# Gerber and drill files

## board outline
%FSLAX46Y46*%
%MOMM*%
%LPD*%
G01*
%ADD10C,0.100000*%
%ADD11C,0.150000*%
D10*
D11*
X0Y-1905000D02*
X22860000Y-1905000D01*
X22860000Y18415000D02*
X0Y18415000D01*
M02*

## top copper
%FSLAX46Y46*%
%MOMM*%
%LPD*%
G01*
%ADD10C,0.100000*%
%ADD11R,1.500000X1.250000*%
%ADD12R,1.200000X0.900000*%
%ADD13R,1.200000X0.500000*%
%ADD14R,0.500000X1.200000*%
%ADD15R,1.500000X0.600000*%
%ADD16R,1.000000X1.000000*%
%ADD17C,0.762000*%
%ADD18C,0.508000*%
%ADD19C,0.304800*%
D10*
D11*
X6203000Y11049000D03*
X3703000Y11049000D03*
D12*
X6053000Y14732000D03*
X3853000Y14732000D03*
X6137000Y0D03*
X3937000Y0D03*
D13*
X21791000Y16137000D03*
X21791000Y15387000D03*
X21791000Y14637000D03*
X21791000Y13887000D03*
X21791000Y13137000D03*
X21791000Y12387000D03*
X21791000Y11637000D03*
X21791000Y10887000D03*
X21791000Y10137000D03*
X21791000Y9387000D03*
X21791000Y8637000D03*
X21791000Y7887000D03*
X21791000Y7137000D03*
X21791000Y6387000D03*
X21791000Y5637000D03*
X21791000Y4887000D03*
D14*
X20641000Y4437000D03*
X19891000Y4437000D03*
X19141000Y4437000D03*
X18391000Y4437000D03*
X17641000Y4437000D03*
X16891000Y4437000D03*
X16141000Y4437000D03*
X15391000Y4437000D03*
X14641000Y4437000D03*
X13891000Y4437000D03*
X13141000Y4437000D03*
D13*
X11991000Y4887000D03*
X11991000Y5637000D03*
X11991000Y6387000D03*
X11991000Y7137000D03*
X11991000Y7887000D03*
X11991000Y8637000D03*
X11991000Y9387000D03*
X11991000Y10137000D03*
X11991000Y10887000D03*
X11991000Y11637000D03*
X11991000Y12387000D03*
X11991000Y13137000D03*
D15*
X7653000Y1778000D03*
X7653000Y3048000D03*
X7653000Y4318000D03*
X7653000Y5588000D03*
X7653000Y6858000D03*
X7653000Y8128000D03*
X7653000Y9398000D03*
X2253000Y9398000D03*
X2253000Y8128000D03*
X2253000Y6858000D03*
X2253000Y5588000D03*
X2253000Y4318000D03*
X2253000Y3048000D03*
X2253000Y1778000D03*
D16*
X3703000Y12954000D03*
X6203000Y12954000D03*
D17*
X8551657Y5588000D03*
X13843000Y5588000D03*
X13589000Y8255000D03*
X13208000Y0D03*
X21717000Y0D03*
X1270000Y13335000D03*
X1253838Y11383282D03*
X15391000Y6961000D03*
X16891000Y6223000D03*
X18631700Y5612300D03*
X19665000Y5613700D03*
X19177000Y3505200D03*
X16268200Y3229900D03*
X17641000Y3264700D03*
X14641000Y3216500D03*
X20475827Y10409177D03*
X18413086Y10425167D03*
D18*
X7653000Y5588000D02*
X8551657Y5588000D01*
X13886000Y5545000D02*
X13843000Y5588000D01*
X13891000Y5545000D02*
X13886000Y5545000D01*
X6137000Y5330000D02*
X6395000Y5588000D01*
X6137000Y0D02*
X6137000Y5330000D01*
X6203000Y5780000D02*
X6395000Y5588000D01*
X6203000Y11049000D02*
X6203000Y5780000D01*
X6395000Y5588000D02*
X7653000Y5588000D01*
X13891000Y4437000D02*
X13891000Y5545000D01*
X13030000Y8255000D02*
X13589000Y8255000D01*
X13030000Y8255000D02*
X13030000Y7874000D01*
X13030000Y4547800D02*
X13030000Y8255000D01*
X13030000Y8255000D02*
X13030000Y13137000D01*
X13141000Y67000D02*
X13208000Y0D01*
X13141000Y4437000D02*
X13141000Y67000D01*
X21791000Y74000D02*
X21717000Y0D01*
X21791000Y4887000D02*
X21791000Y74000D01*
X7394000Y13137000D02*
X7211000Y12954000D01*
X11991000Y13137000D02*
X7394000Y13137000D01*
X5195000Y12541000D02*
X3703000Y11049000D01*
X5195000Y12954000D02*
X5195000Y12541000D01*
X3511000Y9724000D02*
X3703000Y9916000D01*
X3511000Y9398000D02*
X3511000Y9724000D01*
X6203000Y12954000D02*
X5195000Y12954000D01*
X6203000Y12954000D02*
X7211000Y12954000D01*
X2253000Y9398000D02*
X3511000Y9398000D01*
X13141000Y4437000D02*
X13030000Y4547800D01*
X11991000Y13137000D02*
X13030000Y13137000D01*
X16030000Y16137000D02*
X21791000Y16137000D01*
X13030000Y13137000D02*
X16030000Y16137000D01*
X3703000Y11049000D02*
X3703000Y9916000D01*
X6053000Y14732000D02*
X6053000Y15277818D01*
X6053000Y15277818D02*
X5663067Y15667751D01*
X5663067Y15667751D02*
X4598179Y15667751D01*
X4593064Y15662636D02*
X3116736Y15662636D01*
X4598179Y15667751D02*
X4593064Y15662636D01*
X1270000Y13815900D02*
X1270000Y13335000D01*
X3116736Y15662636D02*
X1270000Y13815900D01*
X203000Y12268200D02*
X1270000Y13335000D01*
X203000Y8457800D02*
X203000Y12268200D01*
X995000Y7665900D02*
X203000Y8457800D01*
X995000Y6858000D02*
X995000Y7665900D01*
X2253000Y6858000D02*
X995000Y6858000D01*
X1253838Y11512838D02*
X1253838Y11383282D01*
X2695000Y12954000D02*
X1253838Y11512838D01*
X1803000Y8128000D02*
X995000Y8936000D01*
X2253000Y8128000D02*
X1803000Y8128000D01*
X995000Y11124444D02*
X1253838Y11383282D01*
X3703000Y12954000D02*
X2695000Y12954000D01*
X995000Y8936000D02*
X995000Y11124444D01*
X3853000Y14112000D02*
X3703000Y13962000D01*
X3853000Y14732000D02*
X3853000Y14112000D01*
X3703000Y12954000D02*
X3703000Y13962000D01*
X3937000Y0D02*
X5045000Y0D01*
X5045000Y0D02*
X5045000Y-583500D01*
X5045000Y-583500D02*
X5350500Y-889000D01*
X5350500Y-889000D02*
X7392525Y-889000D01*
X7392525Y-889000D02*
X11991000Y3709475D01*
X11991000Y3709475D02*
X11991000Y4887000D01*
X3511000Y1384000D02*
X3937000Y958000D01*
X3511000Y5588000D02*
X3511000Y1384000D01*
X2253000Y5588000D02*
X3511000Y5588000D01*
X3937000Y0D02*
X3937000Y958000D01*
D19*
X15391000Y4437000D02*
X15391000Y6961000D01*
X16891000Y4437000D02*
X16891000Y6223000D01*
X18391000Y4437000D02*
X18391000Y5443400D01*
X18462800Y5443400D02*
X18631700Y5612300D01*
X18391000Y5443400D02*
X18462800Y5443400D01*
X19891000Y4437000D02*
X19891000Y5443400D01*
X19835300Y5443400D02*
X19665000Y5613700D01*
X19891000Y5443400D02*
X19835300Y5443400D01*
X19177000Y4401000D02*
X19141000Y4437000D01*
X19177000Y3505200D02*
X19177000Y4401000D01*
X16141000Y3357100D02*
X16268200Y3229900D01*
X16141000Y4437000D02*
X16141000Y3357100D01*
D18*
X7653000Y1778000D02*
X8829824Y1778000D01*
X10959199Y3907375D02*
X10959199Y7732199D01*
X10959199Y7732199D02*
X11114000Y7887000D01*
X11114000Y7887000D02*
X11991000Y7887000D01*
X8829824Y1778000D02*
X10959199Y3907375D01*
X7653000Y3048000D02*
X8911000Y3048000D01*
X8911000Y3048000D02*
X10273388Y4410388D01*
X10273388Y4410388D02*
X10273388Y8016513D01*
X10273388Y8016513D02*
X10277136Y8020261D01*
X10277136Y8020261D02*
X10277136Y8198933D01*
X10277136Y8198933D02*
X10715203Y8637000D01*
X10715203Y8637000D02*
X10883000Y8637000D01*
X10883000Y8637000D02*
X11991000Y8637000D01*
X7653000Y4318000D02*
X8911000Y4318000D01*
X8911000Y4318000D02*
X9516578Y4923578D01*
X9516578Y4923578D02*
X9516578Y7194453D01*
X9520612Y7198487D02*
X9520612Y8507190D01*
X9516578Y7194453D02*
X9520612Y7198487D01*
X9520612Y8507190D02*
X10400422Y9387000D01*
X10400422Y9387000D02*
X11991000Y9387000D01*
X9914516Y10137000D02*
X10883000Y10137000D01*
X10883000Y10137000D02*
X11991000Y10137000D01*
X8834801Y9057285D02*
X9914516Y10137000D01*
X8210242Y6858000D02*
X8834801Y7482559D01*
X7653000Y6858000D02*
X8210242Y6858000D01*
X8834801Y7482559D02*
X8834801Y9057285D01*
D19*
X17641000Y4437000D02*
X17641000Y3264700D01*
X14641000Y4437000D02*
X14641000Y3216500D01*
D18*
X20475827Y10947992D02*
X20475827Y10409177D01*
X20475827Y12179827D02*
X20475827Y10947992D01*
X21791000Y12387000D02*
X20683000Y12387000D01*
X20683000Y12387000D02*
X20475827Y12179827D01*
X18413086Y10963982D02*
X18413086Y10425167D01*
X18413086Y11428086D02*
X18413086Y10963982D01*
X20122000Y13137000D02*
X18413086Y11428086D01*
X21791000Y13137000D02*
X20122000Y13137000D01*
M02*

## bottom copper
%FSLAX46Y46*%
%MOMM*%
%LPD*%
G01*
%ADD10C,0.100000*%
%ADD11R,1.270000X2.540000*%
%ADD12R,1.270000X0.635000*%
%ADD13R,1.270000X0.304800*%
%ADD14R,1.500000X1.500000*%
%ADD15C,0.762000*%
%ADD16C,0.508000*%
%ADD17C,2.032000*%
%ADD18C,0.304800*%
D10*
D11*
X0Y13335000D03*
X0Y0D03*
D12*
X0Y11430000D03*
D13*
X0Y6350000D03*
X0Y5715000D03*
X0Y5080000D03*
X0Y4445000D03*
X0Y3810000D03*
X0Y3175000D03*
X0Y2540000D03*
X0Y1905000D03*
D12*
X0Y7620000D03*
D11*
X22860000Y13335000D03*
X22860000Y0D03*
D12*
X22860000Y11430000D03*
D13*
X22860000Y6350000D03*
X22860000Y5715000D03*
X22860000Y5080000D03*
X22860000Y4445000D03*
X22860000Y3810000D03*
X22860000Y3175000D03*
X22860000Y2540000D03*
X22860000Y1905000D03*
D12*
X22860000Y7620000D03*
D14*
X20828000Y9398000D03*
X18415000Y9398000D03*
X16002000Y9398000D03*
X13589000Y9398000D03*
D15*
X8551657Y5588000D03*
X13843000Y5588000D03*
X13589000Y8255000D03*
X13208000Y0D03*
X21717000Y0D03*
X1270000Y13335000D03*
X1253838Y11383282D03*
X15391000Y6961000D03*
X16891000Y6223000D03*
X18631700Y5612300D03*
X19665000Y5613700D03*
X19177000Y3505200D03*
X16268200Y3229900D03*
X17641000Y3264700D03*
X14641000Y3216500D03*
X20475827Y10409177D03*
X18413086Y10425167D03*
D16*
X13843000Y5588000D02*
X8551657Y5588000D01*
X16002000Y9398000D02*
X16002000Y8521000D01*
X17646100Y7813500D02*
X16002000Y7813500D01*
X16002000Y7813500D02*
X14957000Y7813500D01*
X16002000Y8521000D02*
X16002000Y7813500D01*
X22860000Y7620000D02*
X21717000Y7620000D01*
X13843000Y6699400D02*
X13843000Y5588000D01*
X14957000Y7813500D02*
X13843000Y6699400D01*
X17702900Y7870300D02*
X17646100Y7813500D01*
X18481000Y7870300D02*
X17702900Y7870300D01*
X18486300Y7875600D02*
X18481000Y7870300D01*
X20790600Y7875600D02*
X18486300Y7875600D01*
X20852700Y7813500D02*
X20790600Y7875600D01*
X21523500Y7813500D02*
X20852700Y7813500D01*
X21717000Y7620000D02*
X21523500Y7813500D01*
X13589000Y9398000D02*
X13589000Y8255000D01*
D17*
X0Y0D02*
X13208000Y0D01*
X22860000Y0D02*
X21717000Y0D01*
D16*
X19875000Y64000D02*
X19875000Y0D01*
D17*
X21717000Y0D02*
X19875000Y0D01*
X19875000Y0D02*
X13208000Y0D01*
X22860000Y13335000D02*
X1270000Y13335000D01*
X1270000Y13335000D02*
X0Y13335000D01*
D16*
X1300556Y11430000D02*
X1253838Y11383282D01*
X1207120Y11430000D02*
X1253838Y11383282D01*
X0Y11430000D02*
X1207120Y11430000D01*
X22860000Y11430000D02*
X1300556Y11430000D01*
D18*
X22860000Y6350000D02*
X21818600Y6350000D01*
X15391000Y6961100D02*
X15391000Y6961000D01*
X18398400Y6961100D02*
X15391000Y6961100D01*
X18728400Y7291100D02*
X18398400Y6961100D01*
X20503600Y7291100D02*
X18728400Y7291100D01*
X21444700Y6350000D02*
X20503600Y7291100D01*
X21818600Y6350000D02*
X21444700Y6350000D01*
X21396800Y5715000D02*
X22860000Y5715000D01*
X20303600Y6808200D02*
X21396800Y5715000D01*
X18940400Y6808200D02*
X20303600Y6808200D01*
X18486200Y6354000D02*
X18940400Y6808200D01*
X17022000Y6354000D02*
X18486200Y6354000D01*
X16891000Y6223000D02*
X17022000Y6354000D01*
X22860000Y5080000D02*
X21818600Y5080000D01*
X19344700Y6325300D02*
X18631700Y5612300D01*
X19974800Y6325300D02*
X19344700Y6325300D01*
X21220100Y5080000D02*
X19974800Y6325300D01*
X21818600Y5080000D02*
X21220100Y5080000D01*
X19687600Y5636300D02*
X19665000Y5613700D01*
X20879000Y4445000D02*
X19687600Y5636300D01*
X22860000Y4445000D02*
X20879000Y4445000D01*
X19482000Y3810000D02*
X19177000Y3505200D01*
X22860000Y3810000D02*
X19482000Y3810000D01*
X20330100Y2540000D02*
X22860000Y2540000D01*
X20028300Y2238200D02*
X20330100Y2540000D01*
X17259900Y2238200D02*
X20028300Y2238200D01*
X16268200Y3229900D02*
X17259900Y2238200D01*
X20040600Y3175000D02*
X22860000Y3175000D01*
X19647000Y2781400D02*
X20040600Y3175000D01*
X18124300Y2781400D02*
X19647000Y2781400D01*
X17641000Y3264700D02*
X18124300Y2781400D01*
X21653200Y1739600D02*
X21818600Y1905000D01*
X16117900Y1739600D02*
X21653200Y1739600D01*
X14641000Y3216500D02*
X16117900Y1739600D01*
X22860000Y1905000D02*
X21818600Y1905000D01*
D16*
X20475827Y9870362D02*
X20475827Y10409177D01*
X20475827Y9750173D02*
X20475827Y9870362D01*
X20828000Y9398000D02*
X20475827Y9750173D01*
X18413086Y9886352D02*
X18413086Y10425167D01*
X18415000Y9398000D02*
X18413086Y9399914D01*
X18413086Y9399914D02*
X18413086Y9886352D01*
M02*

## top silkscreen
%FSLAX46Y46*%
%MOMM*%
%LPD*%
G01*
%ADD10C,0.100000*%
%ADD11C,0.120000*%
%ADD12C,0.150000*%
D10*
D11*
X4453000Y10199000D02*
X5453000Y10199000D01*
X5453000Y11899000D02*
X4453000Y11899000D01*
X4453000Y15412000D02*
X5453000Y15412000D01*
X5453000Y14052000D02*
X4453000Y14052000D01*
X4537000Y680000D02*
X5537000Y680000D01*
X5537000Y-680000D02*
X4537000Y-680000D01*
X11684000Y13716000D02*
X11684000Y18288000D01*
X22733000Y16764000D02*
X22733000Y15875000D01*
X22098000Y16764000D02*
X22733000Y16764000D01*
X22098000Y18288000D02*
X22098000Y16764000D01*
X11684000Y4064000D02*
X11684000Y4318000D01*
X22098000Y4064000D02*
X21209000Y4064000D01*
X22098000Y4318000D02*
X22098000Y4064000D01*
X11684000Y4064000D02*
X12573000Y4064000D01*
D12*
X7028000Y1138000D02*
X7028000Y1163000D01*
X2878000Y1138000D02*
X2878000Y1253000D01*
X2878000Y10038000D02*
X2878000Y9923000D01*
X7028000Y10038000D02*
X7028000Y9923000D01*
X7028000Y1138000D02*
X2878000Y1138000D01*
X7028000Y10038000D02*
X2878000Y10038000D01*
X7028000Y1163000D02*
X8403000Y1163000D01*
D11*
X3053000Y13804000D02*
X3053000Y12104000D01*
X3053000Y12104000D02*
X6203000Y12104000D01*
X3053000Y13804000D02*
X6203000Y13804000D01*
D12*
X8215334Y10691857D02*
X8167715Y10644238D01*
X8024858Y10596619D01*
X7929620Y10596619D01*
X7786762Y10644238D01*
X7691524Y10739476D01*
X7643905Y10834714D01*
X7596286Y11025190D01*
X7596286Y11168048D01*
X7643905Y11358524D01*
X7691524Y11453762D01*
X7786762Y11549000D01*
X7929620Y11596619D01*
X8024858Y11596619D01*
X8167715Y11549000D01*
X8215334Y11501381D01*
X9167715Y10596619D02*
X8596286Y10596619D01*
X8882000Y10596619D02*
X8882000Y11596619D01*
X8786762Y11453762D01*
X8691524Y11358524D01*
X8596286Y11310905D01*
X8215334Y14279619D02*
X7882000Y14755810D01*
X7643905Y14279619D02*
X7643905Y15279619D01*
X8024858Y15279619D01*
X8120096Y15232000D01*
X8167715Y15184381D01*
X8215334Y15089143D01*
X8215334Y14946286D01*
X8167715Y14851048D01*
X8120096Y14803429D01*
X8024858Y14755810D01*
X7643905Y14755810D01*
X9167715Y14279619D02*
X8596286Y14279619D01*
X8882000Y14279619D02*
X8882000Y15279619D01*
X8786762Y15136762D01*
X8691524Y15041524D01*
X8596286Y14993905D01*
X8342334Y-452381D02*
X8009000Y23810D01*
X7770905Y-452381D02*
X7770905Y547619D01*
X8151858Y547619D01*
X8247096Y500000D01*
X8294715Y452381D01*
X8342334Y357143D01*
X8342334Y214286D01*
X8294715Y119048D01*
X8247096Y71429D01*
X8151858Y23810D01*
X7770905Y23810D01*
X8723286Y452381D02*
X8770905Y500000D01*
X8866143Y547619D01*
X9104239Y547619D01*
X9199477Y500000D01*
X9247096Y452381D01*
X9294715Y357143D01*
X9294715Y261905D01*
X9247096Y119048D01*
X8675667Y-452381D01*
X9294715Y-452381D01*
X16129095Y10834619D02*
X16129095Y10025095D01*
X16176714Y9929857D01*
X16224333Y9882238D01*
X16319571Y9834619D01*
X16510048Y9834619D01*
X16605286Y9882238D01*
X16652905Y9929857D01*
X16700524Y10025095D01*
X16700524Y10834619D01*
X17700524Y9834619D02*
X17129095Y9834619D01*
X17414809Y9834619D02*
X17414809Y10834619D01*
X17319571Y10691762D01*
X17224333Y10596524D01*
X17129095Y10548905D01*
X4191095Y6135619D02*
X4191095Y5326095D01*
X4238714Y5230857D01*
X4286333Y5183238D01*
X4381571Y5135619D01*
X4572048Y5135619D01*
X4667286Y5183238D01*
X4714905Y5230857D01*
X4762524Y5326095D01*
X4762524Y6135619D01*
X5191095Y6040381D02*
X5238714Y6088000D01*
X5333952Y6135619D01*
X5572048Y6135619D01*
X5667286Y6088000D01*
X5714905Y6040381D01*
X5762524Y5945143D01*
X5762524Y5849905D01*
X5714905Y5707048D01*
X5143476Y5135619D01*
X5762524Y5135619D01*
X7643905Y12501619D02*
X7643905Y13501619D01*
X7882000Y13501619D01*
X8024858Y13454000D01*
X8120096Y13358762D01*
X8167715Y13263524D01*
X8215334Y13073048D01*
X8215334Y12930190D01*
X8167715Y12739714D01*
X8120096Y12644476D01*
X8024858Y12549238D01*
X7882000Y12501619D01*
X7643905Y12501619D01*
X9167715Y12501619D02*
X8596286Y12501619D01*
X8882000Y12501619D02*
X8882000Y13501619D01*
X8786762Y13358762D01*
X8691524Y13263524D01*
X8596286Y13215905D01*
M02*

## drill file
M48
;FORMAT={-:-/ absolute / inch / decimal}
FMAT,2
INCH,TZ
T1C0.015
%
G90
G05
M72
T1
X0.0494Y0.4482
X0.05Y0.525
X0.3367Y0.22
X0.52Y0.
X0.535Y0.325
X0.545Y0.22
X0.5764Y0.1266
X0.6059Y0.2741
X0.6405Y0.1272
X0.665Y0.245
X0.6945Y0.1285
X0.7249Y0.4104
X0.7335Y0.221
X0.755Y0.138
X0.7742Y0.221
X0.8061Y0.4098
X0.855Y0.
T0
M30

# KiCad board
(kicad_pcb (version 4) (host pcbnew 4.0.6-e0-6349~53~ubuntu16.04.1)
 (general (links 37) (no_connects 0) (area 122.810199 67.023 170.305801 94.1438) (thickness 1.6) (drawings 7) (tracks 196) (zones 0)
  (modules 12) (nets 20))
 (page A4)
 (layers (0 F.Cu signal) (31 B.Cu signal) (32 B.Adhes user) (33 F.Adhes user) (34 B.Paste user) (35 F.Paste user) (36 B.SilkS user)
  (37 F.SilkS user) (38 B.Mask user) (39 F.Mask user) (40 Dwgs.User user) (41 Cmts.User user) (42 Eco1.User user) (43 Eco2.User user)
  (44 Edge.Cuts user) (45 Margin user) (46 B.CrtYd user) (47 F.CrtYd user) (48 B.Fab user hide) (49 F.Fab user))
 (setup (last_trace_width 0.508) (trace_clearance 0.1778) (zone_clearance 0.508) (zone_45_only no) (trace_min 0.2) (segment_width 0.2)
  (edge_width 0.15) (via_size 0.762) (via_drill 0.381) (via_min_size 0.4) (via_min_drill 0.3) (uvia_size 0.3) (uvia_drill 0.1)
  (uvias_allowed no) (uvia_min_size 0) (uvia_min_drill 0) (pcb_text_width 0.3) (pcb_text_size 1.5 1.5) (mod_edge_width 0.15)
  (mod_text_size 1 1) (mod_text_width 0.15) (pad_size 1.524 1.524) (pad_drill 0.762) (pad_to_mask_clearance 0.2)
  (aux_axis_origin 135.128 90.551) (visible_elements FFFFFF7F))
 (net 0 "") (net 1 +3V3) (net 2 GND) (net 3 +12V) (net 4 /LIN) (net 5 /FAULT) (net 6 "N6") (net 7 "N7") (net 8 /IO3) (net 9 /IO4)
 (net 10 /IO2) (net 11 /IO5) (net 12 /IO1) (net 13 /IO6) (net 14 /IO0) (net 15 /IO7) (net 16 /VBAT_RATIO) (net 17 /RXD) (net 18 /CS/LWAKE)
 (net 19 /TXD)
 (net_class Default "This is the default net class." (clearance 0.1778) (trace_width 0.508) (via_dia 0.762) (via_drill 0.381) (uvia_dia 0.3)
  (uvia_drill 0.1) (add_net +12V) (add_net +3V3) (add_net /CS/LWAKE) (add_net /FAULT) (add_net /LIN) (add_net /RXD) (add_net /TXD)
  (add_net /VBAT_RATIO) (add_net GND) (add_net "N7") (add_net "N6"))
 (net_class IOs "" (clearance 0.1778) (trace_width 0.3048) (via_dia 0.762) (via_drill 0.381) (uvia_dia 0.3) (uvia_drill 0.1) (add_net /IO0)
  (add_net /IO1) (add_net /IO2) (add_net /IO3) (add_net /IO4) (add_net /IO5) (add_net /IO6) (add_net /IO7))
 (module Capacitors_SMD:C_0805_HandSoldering (layer F.Cu) (at 140.081 79.502 180)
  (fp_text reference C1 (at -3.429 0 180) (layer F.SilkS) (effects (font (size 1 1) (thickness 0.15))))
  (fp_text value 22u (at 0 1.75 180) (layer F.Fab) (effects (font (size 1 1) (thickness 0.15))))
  (fp_line (start 0.5 -0.85) (end -0.5 -0.85) (layer F.SilkS) (width 0.12))
  (fp_line (start -0.5 0.85) (end 0.5 0.85) (layer F.SilkS) (width 0.12))
  (pad 1 smd rect (at -1.25 0 180) (size 1.5 1.25) (layers F.Cu F.Paste F.Mask) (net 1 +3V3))
  (pad 2 smd rect (at 1.25 0 180) (size 1.5 1.25) (layers F.Cu F.Paste F.Mask) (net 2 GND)))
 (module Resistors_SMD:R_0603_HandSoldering (layer F.Cu) (at 140.081 75.819 180)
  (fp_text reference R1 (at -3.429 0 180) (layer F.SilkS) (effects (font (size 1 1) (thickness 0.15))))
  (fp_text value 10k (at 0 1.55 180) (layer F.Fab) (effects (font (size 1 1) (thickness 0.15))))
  (fp_line (start 0.5 0.68) (end -0.5 0.68) (layer F.SilkS) (width 0.12))
  (fp_line (start -0.5 -0.68) (end 0.5 -0.68) (layer F.SilkS) (width 0.12))
  (pad 1 smd rect (at -1.1 0 180) (size 1.2 0.9) (layers F.Cu F.Paste F.Mask) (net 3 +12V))
  (pad 2 smd rect (at 1.1 0 180) (size 1.2 0.9) (layers F.Cu F.Paste F.Mask) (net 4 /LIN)))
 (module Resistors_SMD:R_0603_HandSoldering (layer F.Cu) (at 140.165 90.551 180)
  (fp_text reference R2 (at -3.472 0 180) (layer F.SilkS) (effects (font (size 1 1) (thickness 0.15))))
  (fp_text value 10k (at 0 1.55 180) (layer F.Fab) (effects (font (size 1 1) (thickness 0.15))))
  (fp_line (start 0.5 0.68) (end -0.5 0.68) (layer F.SilkS) (width 0.12))
  (fp_line (start -0.5 -0.68) (end 0.5 -0.68) (layer F.SilkS) (width 0.12))
  (pad 1 smd rect (at -1.1 0 180) (size 1.2 0.9) (layers F.Cu F.Paste F.Mask) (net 1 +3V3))
  (pad 2 smd rect (at 1.1 0 180) (size 1.2 0.9) (layers F.Cu F.Paste F.Mask) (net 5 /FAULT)))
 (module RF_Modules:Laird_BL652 (layer F.Cu) (at 152.019 80.264 270)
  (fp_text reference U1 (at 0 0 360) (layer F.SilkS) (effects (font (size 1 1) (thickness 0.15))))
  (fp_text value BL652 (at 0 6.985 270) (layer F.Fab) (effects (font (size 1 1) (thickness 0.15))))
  (fp_line (start -3.429 5.207) (end -8.001 5.207) (layer F.SilkS) (width 0.12))
  (fp_line (start -6.477 -5.842) (end -5.588 -5.842) (layer F.SilkS) (width 0.12))
  (fp_line (start -6.477 -5.207) (end -6.477 -5.842) (layer F.SilkS) (width 0.12))
  (fp_line (start -8.001 -5.207) (end -6.477 -5.207) (layer F.SilkS) (width 0.12))
  (fp_line (start 6.223 5.207) (end 5.969 5.207) (layer F.SilkS) (width 0.12))
  (fp_line (start 6.223 -5.207) (end 6.223 -4.318) (layer F.SilkS) (width 0.12))
  (fp_line (start 5.969 -5.207) (end 6.223 -5.207) (layer F.SilkS) (width 0.12))
  (fp_line (start 6.223 5.207) (end 6.223 4.318) (layer F.SilkS) (width 0.12))
  (pad 1 smd rect (at -5.85 -4.9) (size 1.2 0.5) (layers F.Cu F.Paste F.Mask) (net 2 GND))
  (pad 2 smd rect (at -5.1 -4.9) (size 1.2 0.5) (layers F.Cu F.Paste F.Mask))
  (pad 3 smd rect (at -4.35 -4.9) (size 1.2 0.5) (layers F.Cu F.Paste F.Mask))
  (pad 4 smd rect (at -3.6 -4.9) (size 1.2 0.5) (layers F.Cu F.Paste F.Mask))
  (pad 5 smd rect (at -2.85 -4.9) (size 1.2 0.5) (layers F.Cu F.Paste F.Mask) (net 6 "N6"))
  (pad 6 smd rect (at -2.1 -4.9) (size 1.2 0.5) (layers F.Cu F.Paste F.Mask) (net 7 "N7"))
  (pad 7 smd rect (at -1.35 -4.9) (size 1.2 0.5) (layers F.Cu F.Paste F.Mask))
  (pad 8 smd rect (at -0.6 -4.9) (size 1.2 0.5) (layers F.Cu F.Paste F.Mask))
  (pad 9 smd rect (at 0.15 -4.9) (size 1.2 0.5) (layers F.Cu F.Paste F.Mask))
  (pad 10 smd rect (at 0.9 -4.9) (size 1.2 0.5) (layers F.Cu F.Paste F.Mask))
  (pad 11 smd rect (at 1.65 -4.9) (size 1.2 0.5) (layers F.Cu F.Paste F.Mask))
  (pad 12 smd rect (at 2.4 -4.9) (size 1.2 0.5) (layers F.Cu F.Paste F.Mask))
  (pad 13 smd rect (at 3.15 -4.9) (size 1.2 0.5) (layers F.Cu F.Paste F.Mask))
  (pad 14 smd rect (at 3.9 -4.9) (size 1.2 0.5) (layers F.Cu F.Paste F.Mask))
  (pad 15 smd rect (at 4.65 -4.9) (size 1.2 0.5) (layers F.Cu F.Paste F.Mask))
  (pad 16 smd rect (at 5.4 -4.9) (size 1.2 0.5) (layers F.Cu F.Paste F.Mask) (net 2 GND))
  (pad 17 smd rect (at 5.85 -3.75 270) (size 1.2 0.5) (layers F.Cu F.Paste F.Mask))
  (pad 18 smd rect (at 5.85 -3 270) (size 1.2 0.5) (layers F.Cu F.Paste F.Mask) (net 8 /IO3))
  (pad 19 smd rect (at 5.85 -2.25 270) (size 1.2 0.5) (layers F.Cu F.Paste F.Mask) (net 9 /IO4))
  (pad 20 smd rect (at 5.85 -1.5 270) (size 1.2 0.5) (layers F.Cu F.Paste F.Mask) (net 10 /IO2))
  (pad 21 smd rect (at 5.85 -0.75 270) (size 1.2 0.5) (layers F.Cu F.Paste F.Mask) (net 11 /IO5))
  (pad 22 smd rect (at 5.85 0 270) (size 1.2 0.5) (layers F.Cu F.Paste F.Mask) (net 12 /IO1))
  (pad 23 smd rect (at 5.85 0.75 270) (size 1.2 0.5) (layers F.Cu F.Paste F.Mask) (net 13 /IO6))
  (pad 24 smd rect (at 5.85 1.5 270) (size 1.2 0.5) (layers F.Cu F.Paste F.Mask) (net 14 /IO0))
  (pad 25 smd rect (at 5.85 2.25 270) (size 1.2 0.5) (layers F.Cu F.Paste F.Mask) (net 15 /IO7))
  (pad 26 smd rect (at 5.85 3 270) (size 1.2 0.5) (layers F.Cu F.Paste F.Mask) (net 1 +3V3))
  (pad 27 smd rect (at 5.85 3.75 270) (size 1.2 0.5) (layers F.Cu F.Paste F.Mask) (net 2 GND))
  (pad 28 smd rect (at 5.4 4.9) (size 1.2 0.5) (layers F.Cu F.Paste F.Mask) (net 5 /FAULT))
  (pad 29 smd rect (at 4.65 4.9) (size 1.2 0.5) (layers F.Cu F.Paste F.Mask))
  (pad 30 smd rect (at 3.9 4.9) (size 1.2 0.5) (layers F.Cu F.Paste F.Mask))
  (pad 31 smd rect (at 3.15 4.9) (size 1.2 0.5) (layers F.Cu F.Paste F.Mask))
  (pad 32 smd rect (at 2.4 4.9) (size 1.2 0.5) (layers F.Cu F.Paste F.Mask) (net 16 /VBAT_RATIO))
  (pad 33 smd rect (at 1.65 4.9) (size 1.2 0.5) (layers F.Cu F.Paste F.Mask) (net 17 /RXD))
  (pad 34 smd rect (at 0.9 4.9) (size 1.2 0.5) (layers F.Cu F.Paste F.Mask) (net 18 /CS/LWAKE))
  (pad 35 smd rect (at 0.15 4.9) (size 1.2 0.5) (layers F.Cu F.Paste F.Mask) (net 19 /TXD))
  (pad 36 smd rect (at -0.6 4.9) (size 1.2 0.5) (layers F.Cu F.Paste F.Mask))
  (pad 37 smd rect (at -1.35 4.9) (size 1.2 0.5) (layers F.Cu F.Paste F.Mask))
  (pad 38 smd rect (at -2.1 4.9) (size 1.2 0.5) (layers F.Cu F.Paste F.Mask))
  (pad 39 smd rect (at -2.85 4.9) (size 1.2 0.5) (layers F.Cu F.Paste F.Mask) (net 2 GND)))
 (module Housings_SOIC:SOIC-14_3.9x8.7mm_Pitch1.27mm (layer F.Cu) (at 140.081 84.963 180)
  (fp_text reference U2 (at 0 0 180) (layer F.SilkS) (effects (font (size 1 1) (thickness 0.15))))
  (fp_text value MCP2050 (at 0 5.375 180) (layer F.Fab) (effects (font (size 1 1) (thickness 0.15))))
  (fp_line (start -2.075 -4.45) (end -2.075 -4.425) (layer F.SilkS) (width 0.15))
  (fp_line (start 2.075 -4.45) (end 2.075 -4.335) (layer F.SilkS) (width 0.15))
  (fp_line (start 2.075 4.45) (end 2.075 4.335) (layer F.SilkS) (width 0.15))
  (fp_line (start -2.075 4.45) (end -2.075 4.335) (layer F.SilkS) (width 0.15))
  (fp_line (start -2.075 -4.45) (end 2.075 -4.45) (layer F.SilkS) (width 0.15))
  (fp_line (start -2.075 4.45) (end 2.075 4.45) (layer F.SilkS) (width 0.15))
  (fp_line (start -2.075 -4.425) (end -3.45 -4.425) (layer F.SilkS) (width 0.15))
  (pad 1 smd rect (at -2.7 -3.81 180) (size 1.5 0.6) (layers F.Cu F.Paste F.Mask) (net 16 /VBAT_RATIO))
  (pad 2 smd rect (at -2.7 -2.54 180) (size 1.5 0.6) (layers F.Cu F.Paste F.Mask) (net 17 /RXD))
  (pad 3 smd rect (at -2.7 -1.27 180) (size 1.5 0.6) (layers F.Cu F.Paste F.Mask) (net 18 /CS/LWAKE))
  (pad 4 smd rect (at -2.7 0 180) (size 1.5 0.6) (layers F.Cu F.Paste F.Mask) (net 1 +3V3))
  (pad 5 smd rect (at -2.7 1.27 180) (size 1.5 0.6) (layers F.Cu F.Paste F.Mask) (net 19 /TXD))
  (pad 6 smd rect (at -2.7 2.54 180) (size 1.5 0.6) (layers F.Cu F.Paste F.Mask))
  (pad 7 smd rect (at -2.7 3.81 180) (size 1.5 0.6) (layers F.Cu F.Paste F.Mask))
  (pad 8 smd rect (at 2.7 3.81 180) (size 1.5 0.6) (layers F.Cu F.Paste F.Mask) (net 2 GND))
  (pad 9 smd rect (at 2.7 2.54 180) (size 1.5 0.6) (layers F.Cu F.Paste F.Mask) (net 4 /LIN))
  (pad 10 smd rect (at 2.7 1.27 180) (size 1.5 0.6) (layers F.Cu F.Paste F.Mask) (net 3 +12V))
  (pad 11 smd rect (at 2.7 0 180) (size 1.5 0.6) (layers F.Cu F.Paste F.Mask) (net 5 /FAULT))
  (pad 12 smd rect (at 2.7 -1.27 180) (size 1.5 0.6) (layers F.Cu F.Paste F.Mask))
  (pad 13 smd rect (at 2.7 -2.54 180) (size 1.5 0.6) (layers F.Cu F.Paste F.Mask))
  (pad 14 smd rect (at 2.7 -3.81 180) (size 1.5 0.6) (layers F.Cu F.Paste F.Mask)))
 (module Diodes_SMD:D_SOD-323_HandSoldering (layer F.Cu) (at 140.081 77.597)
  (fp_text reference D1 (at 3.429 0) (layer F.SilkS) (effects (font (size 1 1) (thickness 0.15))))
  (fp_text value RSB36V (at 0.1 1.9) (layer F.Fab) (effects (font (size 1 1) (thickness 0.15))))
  (fp_line (start -1.9 -0.85) (end -1.9 0.85) (layer F.SilkS) (width 0.12))
  (fp_line (start -1.9 0.85) (end 1.25 0.85) (layer F.SilkS) (width 0.12))
  (fp_line (start -1.9 -0.85) (end 1.25 -0.85) (layer F.SilkS) (width 0.12))
  (pad 1 smd rect (at -1.25 0) (size 1 1) (layers F.Cu F.Paste F.Mask) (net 4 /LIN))
  (pad 2 smd rect (at 1.25 0) (size 1 1) (layers F.Cu F.Paste F.Mask) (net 2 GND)))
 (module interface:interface (layer F.Cu) (at 135.128 72.771)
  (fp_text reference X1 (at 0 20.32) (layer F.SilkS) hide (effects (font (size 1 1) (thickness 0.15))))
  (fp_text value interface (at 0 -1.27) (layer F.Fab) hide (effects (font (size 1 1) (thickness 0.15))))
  (pad 1 smd rect (at 0 4.445) (size 1.27 2.54) (layers B.Cu) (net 3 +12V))
  (pad 2 smd rect (at 0 17.78) (size 1.27 2.54) (layers B.Cu) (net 2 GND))
  (pad 3 smd rect (at 0 6.35) (size 1.27 0.635) (layers B.Cu) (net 4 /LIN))
  (pad 5 smd rect (at 0 11.43) (size 1.27 0.3048) (layers B.Cu))
  (pad 6 smd rect (at 0 12.065) (size 1.27 0.3048) (layers B.Cu))
  (pad 7 smd rect (at 0 12.7) (size 1.27 0.3048) (layers B.Cu))
  (pad 8 smd rect (at 0 13.335) (size 1.27 0.3048) (layers B.Cu))
  (pad 9 smd rect (at 0 13.97) (size 1.27 0.3048) (layers B.Cu))
  (pad 10 smd rect (at 0 14.605) (size 1.27 0.3048) (layers B.Cu))
  (pad 11 smd rect (at 0 15.24) (size 1.27 0.3048) (layers B.Cu))
  (pad 12 smd rect (at 0 15.875) (size 1.27 0.3048) (layers B.Cu))
  (pad 4 smd rect (at 0 10.16) (size 1.27 0.635) (layers B.Cu)))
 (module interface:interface (layer F.Cu) (at 157.988 72.771)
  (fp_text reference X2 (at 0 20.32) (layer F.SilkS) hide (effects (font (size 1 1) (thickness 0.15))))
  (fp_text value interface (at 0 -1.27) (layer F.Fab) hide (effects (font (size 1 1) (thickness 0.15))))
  (pad 1 smd rect (at 0 4.445) (size 1.27 2.54) (layers B.Cu) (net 3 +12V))
  (pad 2 smd rect (at 0 17.78) (size 1.27 2.54) (layers B.Cu) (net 2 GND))
  (pad 3 smd rect (at 0 6.35) (size 1.27 0.635) (layers B.Cu) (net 4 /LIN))
  (pad 5 smd rect (at 0 11.43) (size 1.27 0.3048) (layers B.Cu) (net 14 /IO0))
  (pad 6 smd rect (at 0 12.065) (size 1.27 0.3048) (layers B.Cu) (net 12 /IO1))
  (pad 7 smd rect (at 0 12.7) (size 1.27 0.3048) (layers B.Cu) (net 10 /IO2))
  (pad 8 smd rect (at 0 13.335) (size 1.27 0.3048) (layers B.Cu) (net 8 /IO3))
  (pad 9 smd rect (at 0 13.97) (size 1.27 0.3048) (layers B.Cu) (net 9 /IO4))
  (pad 10 smd rect (at 0 14.605) (size 1.27 0.3048) (layers B.Cu) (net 11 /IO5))
  (pad 11 smd rect (at 0 15.24) (size 1.27 0.3048) (layers B.Cu) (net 13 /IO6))
  (pad 12 smd rect (at 0 15.875) (size 1.27 0.3048) (layers B.Cu) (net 15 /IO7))
  (pad 4 smd rect (at 0 10.16) (size 1.27 0.635) (layers B.Cu) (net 1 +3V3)))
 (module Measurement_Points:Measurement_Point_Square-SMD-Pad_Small (layer B.Cu) (at 155.956 81.153)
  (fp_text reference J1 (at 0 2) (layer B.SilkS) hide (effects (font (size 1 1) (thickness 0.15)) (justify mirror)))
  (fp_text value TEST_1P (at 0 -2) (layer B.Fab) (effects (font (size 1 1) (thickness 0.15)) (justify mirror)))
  (pad 1 smd rect (at 0 0) (size 1.5 1.5) (layers B.Cu B.Mask) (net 7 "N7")))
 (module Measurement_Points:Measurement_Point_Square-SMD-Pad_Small (layer B.Cu) (at 153.543 81.153)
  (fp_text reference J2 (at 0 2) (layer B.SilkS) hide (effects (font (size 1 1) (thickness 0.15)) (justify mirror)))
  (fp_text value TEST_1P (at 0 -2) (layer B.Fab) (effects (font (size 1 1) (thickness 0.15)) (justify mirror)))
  (pad 1 smd rect (at 0 0) (size 1.5 1.5) (layers B.Cu B.Mask) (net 6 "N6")))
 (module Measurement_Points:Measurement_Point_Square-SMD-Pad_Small (layer B.Cu) (at 151.13 81.153)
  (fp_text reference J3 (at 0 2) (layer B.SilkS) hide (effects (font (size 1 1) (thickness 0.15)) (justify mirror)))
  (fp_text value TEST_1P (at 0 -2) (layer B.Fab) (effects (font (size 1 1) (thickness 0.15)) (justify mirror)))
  (pad 1 smd rect (at 0 0) (size 1.5 1.5) (layers B.Cu B.Mask) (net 1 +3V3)))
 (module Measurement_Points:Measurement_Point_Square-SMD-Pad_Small (layer B.Cu) (at 148.717 81.153)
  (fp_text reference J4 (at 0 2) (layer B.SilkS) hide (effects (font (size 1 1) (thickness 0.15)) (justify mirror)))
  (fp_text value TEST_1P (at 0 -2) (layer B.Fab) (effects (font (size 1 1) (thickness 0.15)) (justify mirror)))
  (pad 1 smd rect (at 0 0) (size 1.5 1.5) (layers B.Cu B.Mask) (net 2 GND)))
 (gr_line (start 135.128 92.456) (end 157.988 92.456) (layer Edge.Cuts) (width 0.15))
 (gr_line (start 157.988 72.136) (end 135.128 72.136) (layer Edge.Cuts) (width 0.15))
 (via (at 143.679657 84.963) (size 0.762) (drill 0.381) (layers F.Cu B.Cu) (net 1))
 (segment (start 148.971 84.963) (end 143.679657 84.963) (width 0.508) (layer B.Cu) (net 1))
 (segment (start 142.781 84.963) (end 143.679657 84.963) (width 0.508) (layer F.Cu) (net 1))
 (segment (start 151.13 81.153) (end 151.13 82.03) (width 0.508) (layer B.Cu) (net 1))
 (segment (start 152.7741 82.7375) (end 151.13 82.7375) (width 0.508) (layer B.Cu) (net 1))
 (segment (start 151.13 82.7375) (end 150.085 82.7375) (width 0.508) (layer B.Cu) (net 1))
 (segment (start 151.13 82.03) (end 151.13 82.7375) (width 0.508) (layer B.Cu) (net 1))
 (via (at 148.971 84.963) (size 0.762) (layers F.Cu B.Cu) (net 1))
 (segment (start 149.014 85.006) (end 148.971 84.963) (width 0.508) (layer F.Cu) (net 1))
 (segment (start 149.019 85.006) (end 149.014 85.006) (width 0.508) (layer F.Cu) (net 1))
 (segment (start 141.265 85.221) (end 141.523 84.963) (width 0.508) (layer F.Cu) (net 1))
 (segment (start 141.265 90.551) (end 141.265 85.221) (width 0.508) (layer F.Cu) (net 1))
 (segment (start 141.331 84.771) (end 141.523 84.963) (width 0.508) (layer F.Cu) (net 1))
 (segment (start 141.331 79.502) (end 141.331 84.771) (width 0.508) (layer F.Cu) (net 1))
 (segment (start 141.523 84.963) (end 142.781 84.963) (width 0.508) (layer F.Cu) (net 1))
 (segment (start 149.019 86.114) (end 149.019 85.006) (width 0.508) (layer F.Cu) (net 1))
 (segment (start 157.988 82.931) (end 156.845 82.931) (width 0.508) (layer B.Cu) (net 1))
 (segment (start 148.971 83.8516) (end 148.971 84.963) (width 0.508) (layer B.Cu) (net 1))
 (segment (start 150.085 82.7375) (end 148.971 83.8516) (width 0.508) (layer B.Cu) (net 1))
 (segment (start 152.8309 82.6807) (end 152.7741 82.7375) (width 0.508) (layer B.Cu) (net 1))
 (segment (start 153.609 82.6807) (end 152.8309 82.6807) (width 0.508) (layer B.Cu) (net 1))
 (segment (start 153.6143 82.6754) (end 153.609 82.6807) (width 0.508) (layer B.Cu) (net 1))
 (segment (start 155.9186 82.6754) (end 153.6143 82.6754) (width 0.508) (layer B.Cu) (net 1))
 (segment (start 155.9807 82.7375) (end 155.9186 82.6754) (width 0.508) (layer B.Cu) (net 1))
 (segment (start 156.6515 82.7375) (end 155.9807 82.7375) (width 0.508) (layer B.Cu) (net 1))
 (segment (start 156.845 82.931) (end 156.6515 82.7375) (width 0.508) (layer B.Cu) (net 1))
 (segment (start 148.158 82.296) (end 148.717 82.296) (width 0.508) (layer F.Cu) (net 2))
 (segment (start 148.717 81.153) (end 148.717 82.296) (width 0.508) (layer B.Cu) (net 2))
 (segment (start 148.158 82.296) (end 148.158 82.677) (width 0.508) (layer F.Cu) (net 2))
 (segment (start 148.158 86.0032) (end 148.158 82.296) (width 0.508) (layer F.Cu) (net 2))
 (segment (start 148.158 82.296) (end 148.158 77.414) (width 0.508) (layer F.Cu) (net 2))
 (via (at 148.717 82.296) (size 0.762) (drill 0.381) (layers F.Cu B.Cu) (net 2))
 (via (at 148.336 90.551) (size 0.762) (layers F.Cu B.Cu) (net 2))
 (via (at 156.845 90.551) (size 0.762) (layers F.Cu B.Cu) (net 2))
 (segment (start 148.269 90.484) (end 148.336 90.551) (width 0.508) (layer F.Cu) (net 2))
 (segment (start 148.269 86.114) (end 148.269 90.484) (width 0.508) (layer F.Cu) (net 2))
 (segment (start 135.128 90.551) (end 148.336 90.551) (width 2.032) (layer B.Cu) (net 2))
 (segment (start 156.919 90.477) (end 156.845 90.551) (width 0.508) (layer F.Cu) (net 2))
 (segment (start 156.919 85.664) (end 156.919 90.477) (width 0.508) (layer F.Cu) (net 2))
 (segment (start 142.522 77.414) (end 142.339 77.597) (width 0.508) (layer F.Cu) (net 2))
 (segment (start 147.119 77.414) (end 142.522 77.414) (width 0.508) (layer F.Cu) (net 2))
 (segment (start 140.323 78.01) (end 138.831 79.502) (width 0.508) (layer F.Cu) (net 2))
 (segment (start 140.323 77.597) (end 140.323 78.01) (width 0.508) (layer F.Cu) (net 2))
 (segment (start 138.639 80.827) (end 138.831 80.635) (width 0.508) (layer F.Cu) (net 2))
 (segment (start 138.639 81.153) (end 138.639 80.827) (width 0.508) (layer F.Cu) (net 2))
 (segment (start 157.988 90.551) (end 156.845 90.551) (width 2.032) (layer B.Cu) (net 2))
 (segment (start 141.331 77.597) (end 140.323 77.597) (width 0.508) (layer F.Cu) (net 2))
 (segment (start 155.003 90.487) (end 155.003 90.551) (width 0.508) (layer B.Cu) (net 2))
 (segment (start 156.845 90.551) (end 155.003 90.551) (width 2.032) (layer B.Cu) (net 2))
 (segment (start 155.003 90.551) (end 148.336 90.551) (width 2.032) (layer B.Cu) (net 2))
 (segment (start 141.331 77.597) (end 142.339 77.597) (width 0.508) (layer F.Cu) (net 2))
 (segment (start 137.381 81.153) (end 138.639 81.153) (width 0.508) (layer F.Cu) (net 2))
 (segment (start 148.269 86.114) (end 148.158 86.0032) (width 0.508) (layer F.Cu) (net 2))
 (segment (start 147.119 77.414) (end 148.158 77.414) (width 0.508) (layer F.Cu) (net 2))
 (segment (start 151.158 74.414) (end 156.919 74.414) (width 0.508) (layer F.Cu) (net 2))
 (segment (start 148.158 77.414) (end 151.158 74.414) (width 0.508) (layer F.Cu) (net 2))
 (segment (start 138.831 79.502) (end 138.831 80.635) (width 0.508) (layer F.Cu) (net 2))
 (segment (start 141.181 75.819) (end 141.181 75.273182) (width 0.508) (layer F.Cu) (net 3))
 (segment (start 141.181 75.273182) (end 140.791067 74.883249) (width 0.508) (layer F.Cu) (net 3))
 (segment (start 140.791067 74.883249) (end 139.726179 74.883249) (width 0.508) (layer F.Cu) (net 3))
 (segment (start 139.721064 74.888364) (end 138.244736 74.888364) (width 0.508) (layer F.Cu) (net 3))
 (segment (start 139.726179 74.883249) (end 139.721064 74.888364) (width 0.508) (layer F.Cu) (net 3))
 (segment (start 136.398 76.7351) (end 136.398 77.216) (width 0.508) (layer F.Cu) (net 3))
 (segment (start 138.244736 74.888364) (end 136.398 76.7351) (width 0.508) (layer F.Cu) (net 3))
 (segment (start 157.988 77.216) (end 136.398 77.216) (width 2.032) (layer B.Cu) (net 3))
 (via (at 136.398 77.216) (size 0.762) (layers F.Cu B.Cu) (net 3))
 (segment (start 136.398 77.216) (end 135.128 77.216) (width 2.032) (layer B.Cu) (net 3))
 (segment (start 135.331 78.2828) (end 136.398 77.216) (width 0.508) (layer F.Cu) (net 3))
 (segment (start 135.331 82.0932) (end 135.331 78.2828) (width 0.508) (layer F.Cu) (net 3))
 (segment (start 136.123 82.8851) (end 135.331 82.0932) (width 0.508) (layer F.Cu) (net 3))
 (segment (start 136.123 83.693) (end 136.123 82.8851) (width 0.508) (layer F.Cu) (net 3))
 (segment (start 137.381 83.693) (end 136.123 83.693) (width 0.508) (layer F.Cu) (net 3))
 (segment (start 136.428556 79.121) (end 136.381838 79.167718) (width 0.508) (layer B.Cu) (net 4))
 (segment (start 136.33512 79.121) (end 136.381838 79.167718) (width 0.508) (layer B.Cu) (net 4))
 (segment (start 135.128 79.121) (end 136.33512 79.121) (width 0.508) (layer B.Cu) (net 4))
 (segment (start 136.381838 79.038162) (end 136.381838 79.167718) (width 0.508) (layer F.Cu) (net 4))
 (segment (start 137.823 77.597) (end 136.381838 79.038162) (width 0.508) (layer F.Cu) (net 4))
 (segment (start 157.988 79.121) (end 136.428556 79.121) (width 0.508) (layer B.Cu) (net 4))
 (segment (start 136.931 82.423) (end 136.123 81.615) (width 0.508) (layer F.Cu) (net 4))
 (segment (start 137.381 82.423) (end 136.931 82.423) (width 0.508) (layer F.Cu) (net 4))
 (segment (start 136.123 79.426556) (end 136.381838 79.167718) (width 0.508) (layer F.Cu) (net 4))
 (segment (start 138.831 77.597) (end 137.823 77.597) (width 0.508) (layer F.Cu) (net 4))
 (via (at 136.381838 79.167718) (size 0.762) (drill 0.381) (layers F.Cu B.Cu) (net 4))
 (segment (start 136.123 81.615) (end 136.123 79.426556) (width 0.508) (layer F.Cu) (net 4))
 (segment (start 138.981 76.439) (end 138.831 76.589) (width 0.508) (layer F.Cu) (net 4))
 (segment (start 138.981 75.819) (end 138.981 76.439) (width 0.508) (layer F.Cu) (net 4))
 (segment (start 138.831 77.597) (end 138.831 76.589) (width 0.508) (layer F.Cu) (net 4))
 (segment (start 139.065 90.551) (end 140.173 90.551) (width 0.508) (layer F.Cu) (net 5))
 (segment (start 140.173 90.551) (end 140.173 91.1345) (width 0.508) (layer F.Cu) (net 5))
 (segment (start 140.173 91.1345) (end 140.4785 91.44) (width 0.508) (layer F.Cu) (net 5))
 (segment (start 140.4785 91.44) (end 142.520525 91.44) (width 0.508) (layer F.Cu) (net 5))
 (segment (start 142.520525 91.44) (end 147.119 86.841525) (width 0.508) (layer F.Cu) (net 5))
 (segment (start 147.119 86.841525) (end 147.119 85.664) (width 0.508) (layer F.Cu) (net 5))
 (segment (start 138.639 89.167) (end 139.065 89.593) (width 0.508) (layer F.Cu) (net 5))
 (segment (start 138.639 84.963) (end 138.639 89.167) (width 0.508) (layer F.Cu) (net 5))
 (segment (start 137.381 84.963) (end 138.639 84.963) (width 0.508) (layer F.Cu) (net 5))
 (segment (start 139.065 90.551) (end 139.065 89.593) (width 0.508) (layer F.Cu) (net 5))
 (via (at 150.519 83.59) (size 0.762) (layers F.Cu B.Cu) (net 14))
 (segment (start 157.988 84.201) (end 156.9466 84.201) (width 0.3048) (layer B.Cu) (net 14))
 (segment (start 150.519 83.5899) (end 150.519 83.59) (width 0.3048) (layer B.Cu) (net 14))
 (segment (start 153.5264 83.5899) (end 150.519 83.5899) (width 0.3048) (layer B.Cu) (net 14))
 (segment (start 153.8564 83.2599) (end 153.5264 83.5899) (width 0.3048) (layer B.Cu) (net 14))
 (segment (start 155.6316 83.2599) (end 153.8564 83.2599) (width 0.3048) (layer B.Cu) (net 14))
 (segment (start 156.5727 84.201) (end 155.6316 83.2599) (width 0.3048) (layer B.Cu) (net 14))
 (segment (start 156.9466 84.201) (end 156.5727 84.201) (width 0.3048) (layer B.Cu) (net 14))
 (segment (start 150.519 86.114) (end 150.519 83.59) (width 0.3048) (layer F.Cu) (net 14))
 (via (at 152.019 84.328) (size 0.762) (layers F.Cu B.Cu) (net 12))
 (segment (start 152.019 86.114) (end 152.019 84.328) (width 0.3048) (layer F.Cu) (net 12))
 (segment (start 156.5248 84.836) (end 157.988 84.836) (width 0.3048) (layer B.Cu) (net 12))
 (segment (start 155.4316 83.7428) (end 156.5248 84.836) (width 0.3048) (layer B.Cu) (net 12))
 (segment (start 154.0684 83.7428) (end 155.4316 83.7428) (width 0.3048) (layer B.Cu) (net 12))
 (segment (start 153.6142 84.197) (end 154.0684 83.7428) (width 0.3048) (layer B.Cu) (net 12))
 (segment (start 152.15 84.197) (end 153.6142 84.197) (width 0.3048) (layer B.Cu) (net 12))
 (segment (start 152.019 84.328) (end 152.15 84.197) (width 0.3048) (layer B.Cu) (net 12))
 (via (at 153.7597 84.9387) (size 0.762) (layers F.Cu B.Cu) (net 10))
 (segment (start 157.988 85.471) (end 156.9466 85.471) (width 0.3048) (layer B.Cu) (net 10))
 (segment (start 153.519 86.114) (end 153.519 85.1076) (width 0.3048) (layer F.Cu) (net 10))
 (segment (start 154.4727 84.2257) (end 153.7597 84.9387) (width 0.3048) (layer B.Cu) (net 10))
 (segment (start 155.1028 84.2257) (end 154.4727 84.2257) (width 0.3048) (layer B.Cu) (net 10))
 (segment (start 156.3481 85.471) (end 155.1028 84.2257) (width 0.3048) (layer B.Cu) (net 10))
 (segment (start 156.9466 85.471) (end 156.3481 85.471) (width 0.3048) (layer B.Cu) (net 10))
 (segment (start 153.5908 85.1076) (end 153.7597 84.9387) (width 0.3048) (layer F.Cu) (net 10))
 (segment (start 153.519 85.1076) (end 153.5908 85.1076) (width 0.3048) (layer F.Cu) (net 10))
 (via (at 154.793 84.9373) (size 0.762) (layers F.Cu B.Cu) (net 8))
 (segment (start 155.019 86.114) (end 155.019 85.1076) (width 0.3048) (layer F.Cu) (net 8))
 (segment (start 154.8156 84.9147) (end 154.793 84.9373) (width 0.3048) (layer B.Cu) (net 8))
 (segment (start 156.007 86.106) (end 154.8156 84.9147) (width 0.3048) (layer B.Cu) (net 8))
 (segment (start 157.988 86.106) (end 156.007 86.106) (width 0.3048) (layer B.Cu) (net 8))
 (segment (start 154.9633 85.1076) (end 154.793 84.9373) (width 0.3048) (layer F.Cu) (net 8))
 (segment (start 155.019 85.1076) (end 154.9633 85.1076) (width 0.3048) (layer F.Cu) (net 8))
 (via (at 154.305 87.0458) (size 0.762) (layers F.Cu B.Cu) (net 9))
 (segment (start 154.305 86.15) (end 154.269 86.114) (width 0.3048) (layer F.Cu) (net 9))
 (segment (start 154.305 87.0458) (end 154.305 86.15) (width 0.3048) (layer F.Cu) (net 9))
 (segment (start 154.61 86.741) (end 154.305 87.0458) (width 0.3048) (layer B.Cu) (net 9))
 (segment (start 157.988 86.741) (end 154.61 86.741) (width 0.3048) (layer B.Cu) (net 9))
 (via (at 151.3962 87.3211) (size 0.762) (layers F.Cu B.Cu) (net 13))
 (segment (start 155.4581 88.011) (end 157.988 88.011) (width 0.3048) (layer B.Cu) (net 13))
 (segment (start 155.1563 88.3128) (end 155.4581 88.011) (width 0.3048) (layer B.Cu) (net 13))
 (segment (start 152.3879 88.3128) (end 155.1563 88.3128) (width 0.3048) (layer B.Cu) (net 13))
 (segment (start 151.3962 87.3211) (end 152.3879 88.3128) (width 0.3048) (layer B.Cu) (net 13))
 (segment (start 151.269 87.1939) (end 151.3962 87.3211) (width 0.3048) (layer F.Cu) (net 13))
 (segment (start 151.269 86.114) (end 151.269 87.1939) (width 0.3048) (layer F.Cu) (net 13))
 (segment (start 142.781 88.773) (end 143.957824 88.773) (width 0.508) (layer F.Cu) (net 16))
 (segment (start 146.087199 86.643625) (end 146.087199 82.818801) (width 0.508) (layer F.Cu) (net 16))
 (segment (start 146.087199 82.818801) (end 146.242 82.664) (width 0.508) (layer F.Cu) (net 16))
 (segment (start 146.242 82.664) (end 147.119 82.664) (width 0.508) (layer F.Cu) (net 16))
 (segment (start 143.957824 88.773) (end 146.087199 86.643625) (width 0.508) (layer F.Cu) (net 16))
 (segment (start 142.781 87.503) (end 144.039 87.503) (width 0.508) (layer F.Cu) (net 17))
 (segment (start 144.039 87.503) (end 145.401388 86.140612) (width 0.508) (layer F.Cu) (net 17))
 (segment (start 145.401388 86.140612) (end 145.401388 82.534487) (width 0.508) (layer F.Cu) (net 17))
 (segment (start 145.401388 82.534487) (end 145.405136 82.530739) (width 0.508) (layer F.Cu) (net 17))
 (segment (start 145.405136 82.530739) (end 145.405136 82.352067) (width 0.508) (layer F.Cu) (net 17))
 (segment (start 145.405136 82.352067) (end 145.843203 81.914) (width 0.508) (layer F.Cu) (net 17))
 (segment (start 145.843203 81.914) (end 146.011 81.914) (width 0.508) (layer F.Cu) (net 17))
 (segment (start 146.011 81.914) (end 147.119 81.914) (width 0.508) (layer F.Cu) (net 17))
 (segment (start 142.781 86.233) (end 144.039 86.233) (width 0.508) (layer F.Cu) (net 18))
 (segment (start 144.039 86.233) (end 144.644578 85.627422) (width 0.508) (layer F.Cu) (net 18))
 (segment (start 144.644578 85.627422) (end 144.644578 83.356547) (width 0.508) (layer F.Cu) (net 18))
 (segment (start 144.648612 83.352513) (end 144.648612 82.04381) (width 0.508) (layer F.Cu) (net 18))
 (segment (start 144.644578 83.356547) (end 144.648612 83.352513) (width 0.508) (layer F.Cu) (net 18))
 (segment (start 144.648612 82.04381) (end 145.528422 81.164) (width 0.508) (layer F.Cu) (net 18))
 (segment (start 145.528422 81.164) (end 147.119 81.164) (width 0.508) (layer F.Cu) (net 18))
 (segment (start 145.042516 80.414) (end 146.011 80.414) (width 0.508) (layer F.Cu) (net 19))
 (segment (start 146.011 80.414) (end 147.119 80.414) (width 0.508) (layer F.Cu) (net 19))
 (segment (start 143.962801 81.493715) (end 145.042516 80.414) (width 0.508) (layer F.Cu) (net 19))
 (segment (start 143.338242 83.693) (end 143.962801 83.068441) (width 0.508) (layer F.Cu) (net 19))
 (segment (start 142.781 83.693) (end 143.338242 83.693) (width 0.508) (layer F.Cu) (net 19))
 (segment (start 143.962801 83.068441) (end 143.962801 81.493715) (width 0.508) (layer F.Cu) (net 19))
 (via (at 152.769 87.2863) (size 0.762) (layers F.Cu B.Cu) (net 11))
 (segment (start 152.769 86.114) (end 152.769 87.2863) (width 0.3048) (layer F.Cu) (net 11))
 (segment (start 155.1686 87.376) (end 157.988 87.376) (width 0.3048) (layer B.Cu) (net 11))
 (segment (start 154.775 87.7696) (end 155.1686 87.376) (width 0.3048) (layer B.Cu) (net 11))
 (segment (start 153.2523 87.7696) (end 154.775 87.7696) (width 0.3048) (layer B.Cu) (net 11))
 (segment (start 152.769 87.2863) (end 153.2523 87.7696) (width 0.3048) (layer B.Cu) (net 11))
 (via (at 149.769 87.3345) (size 0.762) (layers F.Cu B.Cu) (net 15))
 (segment (start 149.769 86.114) (end 149.769 87.3345) (width 0.3048) (layer F.Cu) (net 15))
 (segment (start 156.7812 88.8114) (end 156.9466 88.646) (width 0.3048) (layer B.Cu) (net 15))
 (segment (start 151.2459 88.8114) (end 156.7812 88.8114) (width 0.3048) (layer B.Cu) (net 15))
 (segment (start 149.769 87.3345) (end 151.2459 88.8114) (width 0.3048) (layer B.Cu) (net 15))
 (segment (start 157.988 88.646) (end 156.9466 88.646) (width 0.3048) (layer B.Cu) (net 15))
 (segment (start 155.603827 79.603008) (end 155.603827 80.141823) (width 0.508) (layer F.Cu) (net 7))
 (segment (start 155.603827 78.371173) (end 155.603827 79.603008) (width 0.508) (layer F.Cu) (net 7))
 (segment (start 156.919 78.164) (end 155.811 78.164) (width 0.508) (layer F.Cu) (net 7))
 (segment (start 155.811 78.164) (end 155.603827 78.371173) (width 0.508) (layer F.Cu) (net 7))
 (segment (start 155.603827 80.680638) (end 155.603827 80.141823) (width 0.508) (layer B.Cu) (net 7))
 (segment (start 155.603827 80.800827) (end 155.603827 80.680638) (width 0.508) (layer B.Cu) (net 7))
 (segment (start 155.956 81.153) (end 155.603827 80.800827) (width 0.508) (layer B.Cu) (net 7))
 (via (at 155.603827 80.141823) (size 0.762) (drill 0.381) (layers F.Cu B.Cu) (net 7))
 (segment (start 153.541086 79.587018) (end 153.541086 80.125833) (width 0.508) (layer F.Cu) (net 6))
 (segment (start 153.541086 79.122914) (end 153.541086 79.587018) (width 0.508) (layer F.Cu) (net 6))
 (segment (start 155.25 77.414) (end 153.541086 79.122914) (width 0.508) (layer F.Cu) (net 6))
 (segment (start 156.919 77.414) (end 155.25 77.414) (width 0.508) (layer F.Cu) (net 6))
 (segment (start 153.541086 80.664648) (end 153.541086 80.125833) (width 0.508) (layer B.Cu) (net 6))
 (segment (start 153.543 81.153) (end 153.541086 81.151086) (width 0.508) (layer B.Cu) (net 6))
 (segment (start 153.541086 81.151086) (end 153.541086 80.664648) (width 0.508) (layer B.Cu) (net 6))
 (via (at 153.541086 80.125833) (size 0.762) (drill 0.381) (layers F.Cu B.Cu) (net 6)))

